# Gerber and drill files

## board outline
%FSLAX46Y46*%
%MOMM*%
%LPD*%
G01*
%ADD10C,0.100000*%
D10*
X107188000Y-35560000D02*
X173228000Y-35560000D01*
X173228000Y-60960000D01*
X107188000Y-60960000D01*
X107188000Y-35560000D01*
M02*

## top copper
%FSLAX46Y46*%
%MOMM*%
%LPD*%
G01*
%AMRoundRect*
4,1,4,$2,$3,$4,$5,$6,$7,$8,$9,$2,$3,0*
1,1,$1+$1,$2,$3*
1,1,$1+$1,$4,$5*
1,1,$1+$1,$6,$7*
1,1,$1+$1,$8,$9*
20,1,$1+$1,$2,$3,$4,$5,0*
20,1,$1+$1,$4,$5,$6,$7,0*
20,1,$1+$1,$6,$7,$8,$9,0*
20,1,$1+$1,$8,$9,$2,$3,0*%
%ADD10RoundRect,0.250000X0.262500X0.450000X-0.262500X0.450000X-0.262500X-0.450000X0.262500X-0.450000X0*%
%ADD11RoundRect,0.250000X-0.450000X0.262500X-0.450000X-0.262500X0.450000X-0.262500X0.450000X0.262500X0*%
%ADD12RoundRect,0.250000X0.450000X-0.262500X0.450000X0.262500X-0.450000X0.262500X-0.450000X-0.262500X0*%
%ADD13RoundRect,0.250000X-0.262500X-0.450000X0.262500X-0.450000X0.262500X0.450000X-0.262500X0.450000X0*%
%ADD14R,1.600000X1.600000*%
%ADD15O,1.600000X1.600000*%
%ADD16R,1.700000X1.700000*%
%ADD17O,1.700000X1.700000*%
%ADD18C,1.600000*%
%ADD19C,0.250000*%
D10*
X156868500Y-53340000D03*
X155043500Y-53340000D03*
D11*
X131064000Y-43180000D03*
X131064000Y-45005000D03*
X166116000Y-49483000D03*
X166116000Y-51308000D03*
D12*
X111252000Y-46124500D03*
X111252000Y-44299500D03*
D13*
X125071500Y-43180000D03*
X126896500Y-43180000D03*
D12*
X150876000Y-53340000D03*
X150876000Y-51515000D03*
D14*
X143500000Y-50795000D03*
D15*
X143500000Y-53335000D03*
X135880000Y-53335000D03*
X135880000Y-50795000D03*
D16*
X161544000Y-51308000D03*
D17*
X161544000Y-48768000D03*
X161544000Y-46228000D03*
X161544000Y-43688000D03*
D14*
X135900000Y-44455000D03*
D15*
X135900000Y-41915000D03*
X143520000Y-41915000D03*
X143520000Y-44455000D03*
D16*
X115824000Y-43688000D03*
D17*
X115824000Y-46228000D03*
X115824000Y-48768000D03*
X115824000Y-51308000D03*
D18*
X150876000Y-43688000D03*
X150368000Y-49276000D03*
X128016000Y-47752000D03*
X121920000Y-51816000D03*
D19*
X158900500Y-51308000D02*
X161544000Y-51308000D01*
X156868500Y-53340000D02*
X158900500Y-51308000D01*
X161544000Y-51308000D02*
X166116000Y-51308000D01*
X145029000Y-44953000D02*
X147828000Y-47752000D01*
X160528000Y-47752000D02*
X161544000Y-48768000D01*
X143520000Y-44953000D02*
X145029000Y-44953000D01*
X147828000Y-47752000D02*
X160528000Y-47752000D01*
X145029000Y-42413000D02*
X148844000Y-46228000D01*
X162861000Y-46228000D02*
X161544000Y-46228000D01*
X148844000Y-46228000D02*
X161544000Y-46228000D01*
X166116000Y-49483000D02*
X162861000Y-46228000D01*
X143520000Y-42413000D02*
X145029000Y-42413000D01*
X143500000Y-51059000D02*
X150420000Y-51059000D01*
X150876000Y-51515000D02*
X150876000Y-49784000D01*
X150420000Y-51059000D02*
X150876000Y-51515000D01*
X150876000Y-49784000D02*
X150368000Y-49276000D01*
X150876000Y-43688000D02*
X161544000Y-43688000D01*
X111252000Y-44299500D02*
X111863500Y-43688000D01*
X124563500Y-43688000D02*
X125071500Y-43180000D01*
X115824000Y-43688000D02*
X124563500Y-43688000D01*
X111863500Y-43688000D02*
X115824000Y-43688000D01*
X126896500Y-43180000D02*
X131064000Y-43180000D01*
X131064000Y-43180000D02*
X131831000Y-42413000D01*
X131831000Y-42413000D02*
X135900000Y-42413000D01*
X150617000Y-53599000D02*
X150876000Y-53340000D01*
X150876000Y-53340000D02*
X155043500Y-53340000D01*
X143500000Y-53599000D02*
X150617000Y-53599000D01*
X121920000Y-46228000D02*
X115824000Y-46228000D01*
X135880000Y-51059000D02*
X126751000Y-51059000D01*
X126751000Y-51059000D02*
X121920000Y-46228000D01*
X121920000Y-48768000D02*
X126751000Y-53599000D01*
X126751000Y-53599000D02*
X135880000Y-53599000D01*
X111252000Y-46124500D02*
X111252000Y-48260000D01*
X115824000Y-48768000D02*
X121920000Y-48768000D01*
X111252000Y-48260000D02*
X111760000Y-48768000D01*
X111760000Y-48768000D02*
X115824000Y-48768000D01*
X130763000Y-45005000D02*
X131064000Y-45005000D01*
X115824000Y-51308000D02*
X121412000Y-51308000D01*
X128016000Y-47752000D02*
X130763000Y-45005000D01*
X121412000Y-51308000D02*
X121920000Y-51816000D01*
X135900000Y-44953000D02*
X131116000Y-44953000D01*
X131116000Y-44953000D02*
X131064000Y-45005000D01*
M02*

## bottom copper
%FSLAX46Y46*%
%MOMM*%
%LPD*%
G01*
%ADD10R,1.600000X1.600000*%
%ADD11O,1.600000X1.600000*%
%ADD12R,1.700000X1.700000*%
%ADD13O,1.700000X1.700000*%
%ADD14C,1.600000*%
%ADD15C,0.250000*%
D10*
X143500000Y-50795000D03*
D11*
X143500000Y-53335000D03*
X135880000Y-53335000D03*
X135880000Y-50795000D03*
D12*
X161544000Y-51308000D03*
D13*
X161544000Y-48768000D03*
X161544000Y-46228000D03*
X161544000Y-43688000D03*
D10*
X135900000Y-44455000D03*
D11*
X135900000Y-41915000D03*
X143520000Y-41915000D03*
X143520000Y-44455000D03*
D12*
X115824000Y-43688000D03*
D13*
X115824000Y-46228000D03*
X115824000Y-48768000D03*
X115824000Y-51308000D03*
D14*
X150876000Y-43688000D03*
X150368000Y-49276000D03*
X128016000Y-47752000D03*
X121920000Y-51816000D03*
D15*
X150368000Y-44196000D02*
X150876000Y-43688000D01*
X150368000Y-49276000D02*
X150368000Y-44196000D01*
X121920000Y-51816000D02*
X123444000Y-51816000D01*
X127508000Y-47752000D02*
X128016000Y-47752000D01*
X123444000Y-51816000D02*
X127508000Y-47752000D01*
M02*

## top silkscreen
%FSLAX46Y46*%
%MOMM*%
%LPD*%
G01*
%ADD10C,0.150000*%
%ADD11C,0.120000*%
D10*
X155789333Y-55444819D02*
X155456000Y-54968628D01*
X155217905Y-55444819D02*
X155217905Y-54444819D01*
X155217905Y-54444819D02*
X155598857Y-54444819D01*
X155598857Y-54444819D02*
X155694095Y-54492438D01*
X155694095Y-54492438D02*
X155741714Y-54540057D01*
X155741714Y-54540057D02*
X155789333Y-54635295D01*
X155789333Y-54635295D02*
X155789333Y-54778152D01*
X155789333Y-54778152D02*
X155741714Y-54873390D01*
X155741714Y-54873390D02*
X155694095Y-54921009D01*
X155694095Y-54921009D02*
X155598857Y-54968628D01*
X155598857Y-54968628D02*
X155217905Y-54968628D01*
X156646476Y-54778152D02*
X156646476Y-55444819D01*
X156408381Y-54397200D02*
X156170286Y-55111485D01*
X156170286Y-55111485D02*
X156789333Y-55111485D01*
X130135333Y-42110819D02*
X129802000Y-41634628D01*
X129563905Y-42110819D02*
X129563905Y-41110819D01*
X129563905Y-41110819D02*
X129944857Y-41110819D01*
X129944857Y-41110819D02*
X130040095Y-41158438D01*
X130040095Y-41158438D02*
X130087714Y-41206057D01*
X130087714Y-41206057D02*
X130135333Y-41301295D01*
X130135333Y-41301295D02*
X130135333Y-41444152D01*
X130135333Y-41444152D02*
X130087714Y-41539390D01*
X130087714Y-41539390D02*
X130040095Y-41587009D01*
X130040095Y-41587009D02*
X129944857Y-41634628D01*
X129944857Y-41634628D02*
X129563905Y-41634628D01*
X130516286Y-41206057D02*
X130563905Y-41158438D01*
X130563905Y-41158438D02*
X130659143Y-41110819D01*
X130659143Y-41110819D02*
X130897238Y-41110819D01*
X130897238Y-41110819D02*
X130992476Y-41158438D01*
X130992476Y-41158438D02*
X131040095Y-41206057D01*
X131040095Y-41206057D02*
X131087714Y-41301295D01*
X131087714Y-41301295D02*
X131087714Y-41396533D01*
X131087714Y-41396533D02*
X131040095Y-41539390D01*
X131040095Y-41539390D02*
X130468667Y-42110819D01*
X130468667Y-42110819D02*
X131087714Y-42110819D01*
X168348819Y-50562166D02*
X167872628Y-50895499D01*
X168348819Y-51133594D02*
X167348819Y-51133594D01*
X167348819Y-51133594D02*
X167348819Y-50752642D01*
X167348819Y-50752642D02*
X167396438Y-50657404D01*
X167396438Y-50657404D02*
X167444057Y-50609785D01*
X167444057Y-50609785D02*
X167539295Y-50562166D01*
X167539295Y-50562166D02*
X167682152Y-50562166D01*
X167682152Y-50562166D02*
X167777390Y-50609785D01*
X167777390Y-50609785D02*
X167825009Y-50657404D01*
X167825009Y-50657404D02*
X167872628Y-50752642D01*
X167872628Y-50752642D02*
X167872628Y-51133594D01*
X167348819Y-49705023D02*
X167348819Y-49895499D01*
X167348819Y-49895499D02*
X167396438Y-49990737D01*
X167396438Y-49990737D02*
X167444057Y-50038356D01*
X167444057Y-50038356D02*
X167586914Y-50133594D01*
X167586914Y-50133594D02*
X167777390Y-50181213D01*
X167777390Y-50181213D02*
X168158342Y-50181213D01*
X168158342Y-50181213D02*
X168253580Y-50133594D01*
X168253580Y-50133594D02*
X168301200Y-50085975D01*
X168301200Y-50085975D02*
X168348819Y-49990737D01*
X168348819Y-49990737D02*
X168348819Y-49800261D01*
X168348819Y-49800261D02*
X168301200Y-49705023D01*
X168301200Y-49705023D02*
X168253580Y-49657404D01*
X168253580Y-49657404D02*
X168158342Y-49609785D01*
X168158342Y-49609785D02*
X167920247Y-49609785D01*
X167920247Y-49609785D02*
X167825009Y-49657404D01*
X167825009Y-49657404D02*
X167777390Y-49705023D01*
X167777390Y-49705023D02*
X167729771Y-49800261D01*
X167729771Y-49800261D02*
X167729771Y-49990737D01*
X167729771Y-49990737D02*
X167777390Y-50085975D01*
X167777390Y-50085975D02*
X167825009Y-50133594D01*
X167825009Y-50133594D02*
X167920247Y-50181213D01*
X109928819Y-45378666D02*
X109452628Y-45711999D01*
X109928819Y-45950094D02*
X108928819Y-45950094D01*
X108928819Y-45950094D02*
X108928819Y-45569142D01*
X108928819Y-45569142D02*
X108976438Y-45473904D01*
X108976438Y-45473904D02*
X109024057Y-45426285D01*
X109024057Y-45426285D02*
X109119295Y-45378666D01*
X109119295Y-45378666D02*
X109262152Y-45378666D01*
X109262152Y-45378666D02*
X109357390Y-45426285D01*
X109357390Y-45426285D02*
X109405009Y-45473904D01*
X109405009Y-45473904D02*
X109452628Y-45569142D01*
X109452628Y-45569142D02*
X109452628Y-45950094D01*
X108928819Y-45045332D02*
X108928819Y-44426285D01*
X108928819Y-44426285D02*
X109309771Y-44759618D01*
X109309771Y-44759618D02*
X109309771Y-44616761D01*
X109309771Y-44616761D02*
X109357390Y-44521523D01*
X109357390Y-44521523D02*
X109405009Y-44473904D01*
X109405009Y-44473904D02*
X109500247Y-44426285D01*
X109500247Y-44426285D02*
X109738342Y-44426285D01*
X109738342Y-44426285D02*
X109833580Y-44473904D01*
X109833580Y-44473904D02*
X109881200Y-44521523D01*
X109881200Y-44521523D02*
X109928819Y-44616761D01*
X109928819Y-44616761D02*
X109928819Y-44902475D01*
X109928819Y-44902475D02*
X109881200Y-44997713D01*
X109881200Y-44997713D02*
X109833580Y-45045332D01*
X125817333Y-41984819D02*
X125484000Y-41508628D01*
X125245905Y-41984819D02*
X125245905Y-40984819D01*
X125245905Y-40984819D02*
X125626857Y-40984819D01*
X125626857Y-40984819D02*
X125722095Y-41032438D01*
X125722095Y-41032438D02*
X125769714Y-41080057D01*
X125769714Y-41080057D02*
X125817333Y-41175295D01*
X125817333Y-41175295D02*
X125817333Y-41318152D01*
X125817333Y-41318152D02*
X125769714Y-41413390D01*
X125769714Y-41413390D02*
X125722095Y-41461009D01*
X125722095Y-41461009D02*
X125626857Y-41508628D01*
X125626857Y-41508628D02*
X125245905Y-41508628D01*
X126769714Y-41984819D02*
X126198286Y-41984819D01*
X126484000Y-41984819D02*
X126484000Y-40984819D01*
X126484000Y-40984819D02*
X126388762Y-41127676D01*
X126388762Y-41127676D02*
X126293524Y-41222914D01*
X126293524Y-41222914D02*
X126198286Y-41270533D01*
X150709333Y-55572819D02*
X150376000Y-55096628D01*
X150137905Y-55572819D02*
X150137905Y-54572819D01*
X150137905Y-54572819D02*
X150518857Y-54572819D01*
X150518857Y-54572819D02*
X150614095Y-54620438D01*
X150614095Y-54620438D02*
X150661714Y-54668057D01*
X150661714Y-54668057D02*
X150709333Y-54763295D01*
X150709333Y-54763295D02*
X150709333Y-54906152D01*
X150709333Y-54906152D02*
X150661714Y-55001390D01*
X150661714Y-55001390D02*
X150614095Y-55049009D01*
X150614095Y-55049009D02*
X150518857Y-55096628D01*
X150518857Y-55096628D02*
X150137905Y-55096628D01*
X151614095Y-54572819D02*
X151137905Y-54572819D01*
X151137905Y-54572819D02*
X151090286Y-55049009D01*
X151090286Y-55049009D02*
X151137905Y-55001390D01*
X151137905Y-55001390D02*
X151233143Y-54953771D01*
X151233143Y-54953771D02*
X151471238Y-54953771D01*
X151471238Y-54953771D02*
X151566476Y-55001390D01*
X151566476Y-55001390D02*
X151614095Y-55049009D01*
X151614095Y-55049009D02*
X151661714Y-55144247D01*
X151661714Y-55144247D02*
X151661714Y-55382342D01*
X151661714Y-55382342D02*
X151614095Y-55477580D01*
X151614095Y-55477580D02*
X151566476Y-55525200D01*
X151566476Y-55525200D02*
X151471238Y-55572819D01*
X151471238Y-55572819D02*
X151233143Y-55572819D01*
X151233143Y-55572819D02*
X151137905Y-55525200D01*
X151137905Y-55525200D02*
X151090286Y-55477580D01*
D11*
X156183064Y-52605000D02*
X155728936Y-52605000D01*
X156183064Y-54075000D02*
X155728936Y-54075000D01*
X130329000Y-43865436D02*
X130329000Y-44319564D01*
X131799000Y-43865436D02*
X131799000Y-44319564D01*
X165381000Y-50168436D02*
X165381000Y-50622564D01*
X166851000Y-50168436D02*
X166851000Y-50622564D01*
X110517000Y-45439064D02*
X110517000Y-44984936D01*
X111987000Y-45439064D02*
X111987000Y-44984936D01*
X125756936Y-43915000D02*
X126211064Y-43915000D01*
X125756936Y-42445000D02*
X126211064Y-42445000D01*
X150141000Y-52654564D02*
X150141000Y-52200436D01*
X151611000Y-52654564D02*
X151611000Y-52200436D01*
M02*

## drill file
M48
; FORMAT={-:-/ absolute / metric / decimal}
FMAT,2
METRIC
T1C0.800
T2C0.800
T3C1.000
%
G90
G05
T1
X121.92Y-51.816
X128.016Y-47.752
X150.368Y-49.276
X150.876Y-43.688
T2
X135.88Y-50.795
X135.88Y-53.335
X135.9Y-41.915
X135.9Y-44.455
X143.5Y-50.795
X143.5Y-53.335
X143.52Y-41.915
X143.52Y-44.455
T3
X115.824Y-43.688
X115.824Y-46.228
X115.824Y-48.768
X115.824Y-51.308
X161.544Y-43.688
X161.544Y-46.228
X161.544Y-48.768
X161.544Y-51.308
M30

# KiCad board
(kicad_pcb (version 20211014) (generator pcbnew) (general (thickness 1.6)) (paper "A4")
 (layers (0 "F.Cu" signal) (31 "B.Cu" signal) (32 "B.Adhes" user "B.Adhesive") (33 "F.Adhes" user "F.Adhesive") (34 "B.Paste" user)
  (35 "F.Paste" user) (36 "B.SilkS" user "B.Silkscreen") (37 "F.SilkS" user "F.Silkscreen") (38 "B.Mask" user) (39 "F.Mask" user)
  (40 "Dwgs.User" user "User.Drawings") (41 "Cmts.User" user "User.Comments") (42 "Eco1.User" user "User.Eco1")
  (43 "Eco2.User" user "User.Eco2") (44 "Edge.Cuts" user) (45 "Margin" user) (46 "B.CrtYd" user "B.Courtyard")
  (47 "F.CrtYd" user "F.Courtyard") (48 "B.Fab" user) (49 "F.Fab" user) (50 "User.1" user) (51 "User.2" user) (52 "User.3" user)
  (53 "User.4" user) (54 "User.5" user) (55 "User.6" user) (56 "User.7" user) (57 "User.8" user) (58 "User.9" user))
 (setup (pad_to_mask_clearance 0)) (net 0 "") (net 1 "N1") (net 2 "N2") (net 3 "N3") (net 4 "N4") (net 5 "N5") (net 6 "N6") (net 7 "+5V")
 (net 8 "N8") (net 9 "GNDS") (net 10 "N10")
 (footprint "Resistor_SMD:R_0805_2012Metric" (layer "F.Cu") (at 155.956 53.34 180)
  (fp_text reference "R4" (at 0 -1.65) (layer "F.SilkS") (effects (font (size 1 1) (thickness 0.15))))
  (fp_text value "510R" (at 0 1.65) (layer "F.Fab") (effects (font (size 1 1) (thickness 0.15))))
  (fp_line (start -0.227064 0.735) (end 0.227064 0.735) (layer "F.SilkS") (width 0.12))
  (fp_line (start -0.227064 -0.735) (end 0.227064 -0.735) (layer "F.SilkS") (width 0.12))
  (pad "1" smd roundrect (at -0.9125 0 180) (size 1.025 1.4) (layers "F.Cu" "F.Paste" "F.Mask") (roundrect_rratio 0.243902) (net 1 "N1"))
  (pad "2" smd roundrect (at 0.9125 0 180) (size 1.025 1.4) (layers "F.Cu" "F.Paste" "F.Mask") (roundrect_rratio 0.243902) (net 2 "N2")))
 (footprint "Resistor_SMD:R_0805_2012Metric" (layer "F.Cu") (at 131.064 44.0925 -90)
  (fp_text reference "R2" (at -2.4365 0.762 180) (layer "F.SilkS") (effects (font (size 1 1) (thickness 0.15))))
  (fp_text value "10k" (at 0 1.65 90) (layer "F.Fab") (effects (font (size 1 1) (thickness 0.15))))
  (fp_line (start -0.227064 0.735) (end 0.227064 0.735) (layer "F.SilkS") (width 0.12))
  (fp_line (start -0.227064 -0.735) (end 0.227064 -0.735) (layer "F.SilkS") (width 0.12))
  (pad "1" smd roundrect (at -0.9125 0 270) (size 1.025 1.4) (layers "F.Cu" "F.Paste" "F.Mask") (roundrect_rratio 0.243902) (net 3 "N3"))
  (pad "2" smd roundrect (at 0.9125 0 270) (size 1.025 1.4) (layers "F.Cu" "F.Paste" "F.Mask") (roundrect_rratio 0.243902) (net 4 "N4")))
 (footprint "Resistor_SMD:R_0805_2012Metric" (layer "F.Cu") (at 166.116 50.3955 -90)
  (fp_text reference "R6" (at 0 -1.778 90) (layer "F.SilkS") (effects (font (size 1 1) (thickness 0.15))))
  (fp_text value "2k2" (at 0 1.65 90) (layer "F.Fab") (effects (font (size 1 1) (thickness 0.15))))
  (fp_line (start -0.227064 0.735) (end 0.227064 0.735) (layer "F.SilkS") (width 0.12))
  (fp_line (start -0.227064 -0.735) (end 0.227064 -0.735) (layer "F.SilkS") (width 0.12))
  (pad "1" smd roundrect (at -0.9125 0 270) (size 1.025 1.4) (layers "F.Cu" "F.Paste" "F.Mask") (roundrect_rratio 0.243902) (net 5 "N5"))
  (pad "2" smd roundrect (at 0.9125 0 270) (size 1.025 1.4) (layers "F.Cu" "F.Paste" "F.Mask") (roundrect_rratio 0.243902) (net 1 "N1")))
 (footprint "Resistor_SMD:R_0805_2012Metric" (layer "F.Cu") (at 111.252 45.212 90)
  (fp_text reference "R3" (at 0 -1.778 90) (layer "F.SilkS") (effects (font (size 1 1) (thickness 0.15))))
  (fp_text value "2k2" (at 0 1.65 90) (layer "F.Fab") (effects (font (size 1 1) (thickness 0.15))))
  (fp_line (start -0.227064 -0.735) (end 0.227064 -0.735) (layer "F.SilkS") (width 0.12))
  (fp_line (start -0.227064 0.735) (end 0.227064 0.735) (layer "F.SilkS") (width 0.12))
  (pad "1" smd roundrect (at -0.9125 0 90) (size 1.025 1.4) (layers "F.Cu" "F.Paste" "F.Mask") (roundrect_rratio 0.243902) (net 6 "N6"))
  (pad "2" smd roundrect (at 0.9125 0 90) (size 1.025 1.4) (layers "F.Cu" "F.Paste" "F.Mask") (roundrect_rratio 0.243902) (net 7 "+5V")))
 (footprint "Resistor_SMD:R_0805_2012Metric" (layer "F.Cu") (at 125.984 43.18)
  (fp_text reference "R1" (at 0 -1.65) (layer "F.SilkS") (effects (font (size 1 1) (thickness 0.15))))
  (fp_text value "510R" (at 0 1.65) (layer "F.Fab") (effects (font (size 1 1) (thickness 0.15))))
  (fp_line (start -0.227064 0.735) (end 0.227064 0.735) (layer "F.SilkS") (width 0.12))
  (fp_line (start -0.227064 -0.735) (end 0.227064 -0.735) (layer "F.SilkS") (width 0.12))
  (pad "1" smd roundrect (at -0.9125 0) (size 1.025 1.4) (layers "F.Cu" "F.Paste" "F.Mask") (roundrect_rratio 0.243902) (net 7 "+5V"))
  (pad "2" smd roundrect (at 0.9125 0) (size 1.025 1.4) (layers "F.Cu" "F.Paste" "F.Mask") (roundrect_rratio 0.243902) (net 3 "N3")))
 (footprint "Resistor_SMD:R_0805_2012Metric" (layer "F.Cu") (at 150.876 52.4275 90)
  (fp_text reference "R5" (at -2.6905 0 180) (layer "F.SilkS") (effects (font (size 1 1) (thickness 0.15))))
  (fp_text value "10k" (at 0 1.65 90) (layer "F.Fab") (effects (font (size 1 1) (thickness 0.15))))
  (fp_line (start -0.227064 -0.735) (end 0.227064 -0.735) (layer "F.SilkS") (width 0.12))
  (fp_line (start -0.227064 0.735) (end 0.227064 0.735) (layer "F.SilkS") (width 0.12))
  (pad "1" smd roundrect (at -0.9125 0 90) (size 1.025 1.4) (layers "F.Cu" "F.Paste" "F.Mask") (roundrect_rratio 0.243902) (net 2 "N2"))
  (pad "2" smd roundrect (at 0.9125 0 90) (size 1.025 1.4) (layers "F.Cu" "F.Paste" "F.Mask") (roundrect_rratio 0.243902) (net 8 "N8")))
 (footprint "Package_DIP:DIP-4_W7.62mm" (layer "B.Cu") (at 143.5 50.795 180)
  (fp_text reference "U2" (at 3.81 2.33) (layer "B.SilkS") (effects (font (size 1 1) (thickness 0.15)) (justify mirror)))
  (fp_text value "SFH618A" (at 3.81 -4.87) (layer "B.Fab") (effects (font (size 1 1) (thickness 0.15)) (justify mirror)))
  (pad "1" thru_hole rect (at 0 0 180) (size 1.6 1.6) (drill 0.8) (layers *.Cu *.Mask) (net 8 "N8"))
  (pad "2" thru_hole oval (at 0 -2.54 180) (size 1.6 1.6) (drill 0.8) (layers *.Cu *.Mask) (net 8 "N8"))
  (pad "3" thru_hole oval (at 7.62 -2.54 180) (size 1.6 1.6) (drill 0.8) (layers *.Cu *.Mask) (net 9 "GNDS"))
  (pad "4" thru_hole oval (at 7.62 0 180) (size 1.6 1.6) (drill 0.8) (layers *.Cu *.Mask) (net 6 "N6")))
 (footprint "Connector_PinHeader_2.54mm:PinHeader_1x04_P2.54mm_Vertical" (layer "B.Cu") (at 161.544 51.308)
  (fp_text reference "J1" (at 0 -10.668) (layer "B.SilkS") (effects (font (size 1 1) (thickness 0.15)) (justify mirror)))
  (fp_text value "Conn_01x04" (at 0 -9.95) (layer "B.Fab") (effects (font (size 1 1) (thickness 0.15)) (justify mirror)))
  (pad "1" thru_hole rect (at 0 0) (size 1.7 1.7) (drill 1) (layers *.Cu *.Mask) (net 1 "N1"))
  (pad "2" thru_hole oval (at 0 -2.54) (size 1.7 1.7) (drill 1) (layers *.Cu *.Mask) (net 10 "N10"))
  (pad "3" thru_hole oval (at 0 -5.08) (size 1.7 1.7) (drill 1) (layers *.Cu *.Mask) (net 5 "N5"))
  (pad "4" thru_hole oval (at 0 -7.62) (size 1.7 1.7) (drill 1) (layers *.Cu *.Mask) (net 8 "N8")))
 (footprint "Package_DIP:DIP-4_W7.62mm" (layer "B.Cu") (at 135.9 44.455)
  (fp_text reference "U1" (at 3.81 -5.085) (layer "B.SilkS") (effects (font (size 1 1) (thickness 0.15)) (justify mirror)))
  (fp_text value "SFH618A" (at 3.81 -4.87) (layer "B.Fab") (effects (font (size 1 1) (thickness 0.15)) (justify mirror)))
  (pad "1" thru_hole rect (at 0 0) (size 1.6 1.6) (drill 0.8) (layers *.Cu *.Mask) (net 4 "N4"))
  (pad "2" thru_hole oval (at 0 -2.54) (size 1.6 1.6) (drill 0.8) (layers *.Cu *.Mask) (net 4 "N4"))
  (pad "3" thru_hole oval (at 7.62 -2.54) (size 1.6 1.6) (drill 0.8) (layers *.Cu *.Mask) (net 10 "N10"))
  (pad "4" thru_hole oval (at 7.62 0) (size 1.6 1.6) (drill 0.8) (layers *.Cu *.Mask) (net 5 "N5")))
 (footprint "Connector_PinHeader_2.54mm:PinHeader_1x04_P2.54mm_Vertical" (layer "B.Cu") (at 115.824 43.688 180)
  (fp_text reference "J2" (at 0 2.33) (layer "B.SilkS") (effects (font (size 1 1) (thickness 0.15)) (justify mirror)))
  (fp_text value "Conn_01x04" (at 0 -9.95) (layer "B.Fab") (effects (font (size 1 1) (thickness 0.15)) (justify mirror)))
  (pad "1" thru_hole rect (at 0 0 180) (size 1.7 1.7) (drill 1) (layers *.Cu *.Mask) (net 7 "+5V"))
  (pad "2" thru_hole oval (at 0 -2.54 180) (size 1.7 1.7) (drill 1) (layers *.Cu *.Mask) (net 9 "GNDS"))
  (pad "3" thru_hole oval (at 0 -5.08 180) (size 1.7 1.7) (drill 1) (layers *.Cu *.Mask) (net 6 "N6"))
  (pad "4" thru_hole oval (at 0 -7.62 180) (size 1.7 1.7) (drill 1) (layers *.Cu *.Mask) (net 4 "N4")))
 (gr_rect (start 173.228 60.96) (end 107.188 35.56) (layer "Edge.Cuts") (width 0.1) (fill none))
 (segment (start 158.9005 51.308) (end 161.544 51.308) (width 0.25) (layer "F.Cu") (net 1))
 (segment (start 156.8685 53.34) (end 158.9005 51.308) (width 0.25) (layer "F.Cu") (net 1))
 (segment (start 161.544 51.308) (end 166.116 51.308) (width 0.25) (layer "F.Cu") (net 1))
 (segment (start 145.029 44.953) (end 147.828 47.752) (width 0.25) (layer "F.Cu") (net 10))
 (segment (start 160.528 47.752) (end 161.544 48.768) (width 0.25) (layer "F.Cu") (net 10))
 (segment (start 143.52 44.953) (end 145.029 44.953) (width 0.25) (layer "F.Cu") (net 10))
 (segment (start 147.828 47.752) (end 160.528 47.752) (width 0.25) (layer "F.Cu") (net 10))
 (segment (start 145.029 42.413) (end 148.844 46.228) (width 0.25) (layer "F.Cu") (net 5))
 (segment (start 162.861 46.228) (end 161.544 46.228) (width 0.25) (layer "F.Cu") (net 5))
 (segment (start 148.844 46.228) (end 161.544 46.228) (width 0.25) (layer "F.Cu") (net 5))
 (segment (start 166.116 49.483) (end 162.861 46.228) (width 0.25) (layer "F.Cu") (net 5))
 (segment (start 143.52 42.413) (end 145.029 42.413) (width 0.25) (layer "F.Cu") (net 5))
 (segment (start 143.5 51.059) (end 150.42 51.059) (width 0.25) (layer "F.Cu") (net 8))
 (segment (start 150.876 51.515) (end 150.876 49.784) (width 0.25) (layer "F.Cu") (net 8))
 (segment (start 150.42 51.059) (end 150.876 51.515) (width 0.25) (layer "F.Cu") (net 8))
 (segment (start 150.876 49.784) (end 150.368 49.276) (width 0.25) (layer "F.Cu") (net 8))
 (segment (start 150.876 43.688) (end 161.544 43.688) (width 0.25) (layer "F.Cu") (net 8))
 (via (at 150.876 43.688) (size 1.6) (drill 0.8) (layers "F.Cu" "B.Cu") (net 8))
 (via (at 150.368 49.276) (size 1.6) (drill 0.8) (layers "F.Cu" "B.Cu") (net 8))
 (segment (start 150.368 44.196) (end 150.876 43.688) (width 0.25) (layer "B.Cu") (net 8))
 (segment (start 150.368 49.276) (end 150.368 44.196) (width 0.25) (layer "B.Cu") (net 8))
 (segment (start 111.252 44.2995) (end 111.8635 43.688) (width 0.25) (layer "F.Cu") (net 7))
 (segment (start 124.5635 43.688) (end 125.0715 43.18) (width 0.25) (layer "F.Cu") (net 7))
 (segment (start 115.824 43.688) (end 124.5635 43.688) (width 0.25) (layer "F.Cu") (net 7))
 (segment (start 111.8635 43.688) (end 115.824 43.688) (width 0.25) (layer "F.Cu") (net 7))
 (segment (start 126.8965 43.18) (end 131.064 43.18) (width 0.25) (layer "F.Cu") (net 3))
 (segment (start 131.064 43.18) (end 131.831 42.413) (width 0.25) (layer "F.Cu") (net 3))
 (segment (start 131.831 42.413) (end 135.9 42.413) (width 0.25) (layer "F.Cu") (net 3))
 (segment (start 150.617 53.599) (end 150.876 53.34) (width 0.25) (layer "F.Cu") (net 2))
 (segment (start 150.876 53.34) (end 155.0435 53.34) (width 0.25) (layer "F.Cu") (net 2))
 (segment (start 143.5 53.599) (end 150.617 53.599) (width 0.25) (layer "F.Cu") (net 2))
 (segment (start 121.92 46.228) (end 115.824 46.228) (width 0.25) (layer "F.Cu") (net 9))
 (segment (start 135.88 51.059) (end 126.751 51.059) (width 0.25) (layer "F.Cu") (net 9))
 (segment (start 126.751 51.059) (end 121.92 46.228) (width 0.25) (layer "F.Cu") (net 9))
 (segment (start 121.92 48.768) (end 126.751 53.599) (width 0.25) (layer "F.Cu") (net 6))
 (segment (start 126.751 53.599) (end 135.88 53.599) (width 0.25) (layer "F.Cu") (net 6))
 (segment (start 111.252 46.1245) (end 111.252 48.26) (width 0.25) (layer "F.Cu") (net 6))
 (segment (start 115.824 48.768) (end 121.92 48.768) (width 0.25) (layer "F.Cu") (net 6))
 (segment (start 111.252 48.26) (end 111.76 48.768) (width 0.25) (layer "F.Cu") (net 6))
 (segment (start 111.76 48.768) (end 115.824 48.768) (width 0.25) (layer "F.Cu") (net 6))
 (segment (start 130.763 45.005) (end 131.064 45.005) (width 0.25) (layer "F.Cu") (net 4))
 (segment (start 115.824 51.308) (end 121.412 51.308) (width 0.25) (layer "F.Cu") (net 4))
 (segment (start 128.016 47.752) (end 130.763 45.005) (width 0.25) (layer "F.Cu") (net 4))
 (segment (start 121.412 51.308) (end 121.92 51.816) (width 0.25) (layer "F.Cu") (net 4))
 (segment (start 135.9 44.953) (end 131.116 44.953) (width 0.25) (layer "F.Cu") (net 4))
 (segment (start 131.116 44.953) (end 131.064 45.005) (width 0.25) (layer "F.Cu") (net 4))
 (via (at 128.016 47.752) (size 1.6) (drill 0.8) (layers "F.Cu" "B.Cu") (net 4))
 (via (at 121.92 51.816) (size 1.6) (drill 0.8) (layers "F.Cu" "B.Cu") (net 4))
 (segment (start 121.92 51.816) (end 123.444 51.816) (width 0.25) (layer "B.Cu") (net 4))
 (segment (start 127.508 47.752) (end 128.016 47.752) (width 0.25) (layer "B.Cu") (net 4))
 (segment (start 123.444 51.816) (end 127.508 47.752) (width 0.25) (layer "B.Cu") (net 4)))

